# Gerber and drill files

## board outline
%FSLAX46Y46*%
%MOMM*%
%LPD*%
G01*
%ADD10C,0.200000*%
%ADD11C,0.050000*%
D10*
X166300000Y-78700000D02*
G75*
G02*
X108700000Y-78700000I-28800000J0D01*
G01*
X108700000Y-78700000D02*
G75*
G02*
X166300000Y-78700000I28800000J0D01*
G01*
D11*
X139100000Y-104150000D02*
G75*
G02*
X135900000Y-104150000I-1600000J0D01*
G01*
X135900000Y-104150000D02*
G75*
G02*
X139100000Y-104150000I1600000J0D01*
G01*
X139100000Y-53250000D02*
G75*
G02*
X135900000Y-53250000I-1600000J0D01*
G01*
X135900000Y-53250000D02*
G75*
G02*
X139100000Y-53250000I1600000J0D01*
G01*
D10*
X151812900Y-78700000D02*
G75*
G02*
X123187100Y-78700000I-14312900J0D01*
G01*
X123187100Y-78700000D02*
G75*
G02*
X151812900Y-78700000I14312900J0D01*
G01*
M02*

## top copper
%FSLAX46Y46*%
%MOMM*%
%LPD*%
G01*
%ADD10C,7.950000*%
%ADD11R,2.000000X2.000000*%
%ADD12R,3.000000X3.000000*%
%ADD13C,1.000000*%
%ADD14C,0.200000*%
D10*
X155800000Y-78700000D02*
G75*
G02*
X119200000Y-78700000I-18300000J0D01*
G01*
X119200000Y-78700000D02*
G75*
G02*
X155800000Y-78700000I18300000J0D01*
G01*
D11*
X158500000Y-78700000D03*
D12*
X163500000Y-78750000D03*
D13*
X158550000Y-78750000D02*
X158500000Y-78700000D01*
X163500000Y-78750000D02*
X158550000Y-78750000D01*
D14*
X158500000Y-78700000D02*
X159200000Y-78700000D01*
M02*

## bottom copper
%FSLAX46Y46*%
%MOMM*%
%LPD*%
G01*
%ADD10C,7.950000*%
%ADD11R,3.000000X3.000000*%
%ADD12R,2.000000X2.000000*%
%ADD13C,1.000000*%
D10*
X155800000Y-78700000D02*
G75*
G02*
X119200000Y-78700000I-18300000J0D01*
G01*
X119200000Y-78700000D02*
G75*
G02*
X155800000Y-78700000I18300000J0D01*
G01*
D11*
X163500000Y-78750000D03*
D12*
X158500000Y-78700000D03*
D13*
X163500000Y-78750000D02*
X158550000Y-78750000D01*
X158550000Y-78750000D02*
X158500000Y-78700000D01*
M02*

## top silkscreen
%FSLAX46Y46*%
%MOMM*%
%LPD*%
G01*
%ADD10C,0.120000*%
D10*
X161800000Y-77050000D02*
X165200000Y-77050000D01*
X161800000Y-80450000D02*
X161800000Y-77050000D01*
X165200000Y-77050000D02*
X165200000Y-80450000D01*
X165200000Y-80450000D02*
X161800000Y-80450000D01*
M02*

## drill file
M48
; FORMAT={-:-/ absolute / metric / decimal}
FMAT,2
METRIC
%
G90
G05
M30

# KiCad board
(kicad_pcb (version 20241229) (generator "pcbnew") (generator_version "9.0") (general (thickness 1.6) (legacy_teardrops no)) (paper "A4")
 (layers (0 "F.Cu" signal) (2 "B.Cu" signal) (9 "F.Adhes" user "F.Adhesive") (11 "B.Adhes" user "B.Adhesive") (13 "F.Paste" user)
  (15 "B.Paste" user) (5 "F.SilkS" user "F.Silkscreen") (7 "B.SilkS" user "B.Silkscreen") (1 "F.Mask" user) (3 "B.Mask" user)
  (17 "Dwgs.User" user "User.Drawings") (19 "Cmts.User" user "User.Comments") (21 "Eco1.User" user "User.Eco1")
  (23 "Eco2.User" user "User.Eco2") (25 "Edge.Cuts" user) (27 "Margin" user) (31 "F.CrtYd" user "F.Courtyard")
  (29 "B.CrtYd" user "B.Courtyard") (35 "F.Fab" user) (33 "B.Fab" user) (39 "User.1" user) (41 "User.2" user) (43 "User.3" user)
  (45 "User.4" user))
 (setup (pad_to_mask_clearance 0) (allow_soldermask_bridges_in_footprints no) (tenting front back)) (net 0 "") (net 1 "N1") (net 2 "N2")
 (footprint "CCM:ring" (layer "F.Cu") (at 137.5 78.7)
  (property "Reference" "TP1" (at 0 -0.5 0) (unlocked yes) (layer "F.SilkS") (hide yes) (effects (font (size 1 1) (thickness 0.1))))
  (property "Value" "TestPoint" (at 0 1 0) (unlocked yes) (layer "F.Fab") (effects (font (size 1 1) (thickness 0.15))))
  (fp_circle (center 0 0) (end 18.3 0) (stroke (width 7.95) (type solid)) (fill no) (layer "F.Cu"))
  (pad "1" smd rect (at 21 0) (size 2 2) (layers "F.Cu" "F.Mask") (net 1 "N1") (thermal_bridge_angle 45)))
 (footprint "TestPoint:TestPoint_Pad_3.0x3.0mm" (layer "F.Cu") (at 163.5 78.75)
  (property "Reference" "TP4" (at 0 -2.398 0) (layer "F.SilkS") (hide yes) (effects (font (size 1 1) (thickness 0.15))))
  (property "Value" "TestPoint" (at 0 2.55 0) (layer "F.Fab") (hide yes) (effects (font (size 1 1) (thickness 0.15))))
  (fp_line (start -1.7 -1.7) (end 1.7 -1.7) (stroke (width 0.12) (type solid)) (layer "F.SilkS"))
  (fp_line (start -1.7 1.7) (end -1.7 -1.7) (stroke (width 0.12) (type solid)) (layer "F.SilkS"))
  (fp_line (start 1.7 -1.7) (end 1.7 1.7) (stroke (width 0.12) (type solid)) (layer "F.SilkS"))
  (fp_line (start 1.7 1.7) (end -1.7 1.7) (stroke (width 0.12) (type solid)) (layer "F.SilkS"))
  (pad "1" smd rect (at 0 0) (size 3 3) (layers "F.Cu" "F.Mask") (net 1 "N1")))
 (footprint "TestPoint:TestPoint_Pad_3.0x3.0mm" (layer "B.Cu") (at 163.5 78.75 180)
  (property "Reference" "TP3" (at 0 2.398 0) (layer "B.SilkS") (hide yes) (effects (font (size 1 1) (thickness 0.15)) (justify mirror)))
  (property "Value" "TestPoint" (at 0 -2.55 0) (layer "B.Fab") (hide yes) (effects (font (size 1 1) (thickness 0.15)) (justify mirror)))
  (pad "1" smd rect (at 0 0 180) (size 3 3) (layers "B.Cu" "B.Mask") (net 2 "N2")))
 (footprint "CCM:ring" (layer "B.Cu") (at 137.5 78.7)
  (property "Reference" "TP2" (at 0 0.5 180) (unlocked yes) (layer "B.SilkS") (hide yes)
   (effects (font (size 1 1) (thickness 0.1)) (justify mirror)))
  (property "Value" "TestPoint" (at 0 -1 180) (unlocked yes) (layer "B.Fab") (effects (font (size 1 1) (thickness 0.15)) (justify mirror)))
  (fp_circle (center 0 0) (end 18.3 0) (stroke (width 7.95) (type solid)) (fill no) (layer "B.Cu"))
  (pad "1" smd rect (at 21 0) (size 2 2) (layers "B.Cu" "B.Mask") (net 2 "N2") (thermal_bridge_angle 45)))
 (gr_circle (center 137.5 78.7) (end 137.5 107.5) (stroke (width 0.2) (type solid)) (fill no) (layer "Edge.Cuts"))
 (gr_circle (center 137.5 104.15) (end 135.9 104.15) (stroke (width 0.05) (type solid)) (fill no) (layer "Edge.Cuts"))
 (gr_circle (center 137.5 53.25) (end 139.1 53.25) (stroke (width 0.05) (type solid)) (fill no) (layer "Edge.Cuts"))
 (gr_circle (center 137.5 78.7) (end 151.8129 78.7) (stroke (width 0.2) (type solid)) (fill no) (layer "Edge.Cuts"))
 (segment (start 158.55 78.75) (end 158.5 78.7) (width 1) (layer "F.Cu") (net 1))
 (segment (start 163.5 78.75) (end 158.55 78.75) (width 1) (layer "F.Cu") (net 1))
 (segment (start 158.5 78.7) (end 159.2 78.7) (width 0.2) (layer "F.Cu") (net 1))
 (segment (start 163.5 78.75) (end 158.55 78.75) (width 1) (layer "B.Cu") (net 2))
 (segment (start 158.55 78.75) (end 158.5 78.7) (width 1) (layer "B.Cu") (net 2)))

